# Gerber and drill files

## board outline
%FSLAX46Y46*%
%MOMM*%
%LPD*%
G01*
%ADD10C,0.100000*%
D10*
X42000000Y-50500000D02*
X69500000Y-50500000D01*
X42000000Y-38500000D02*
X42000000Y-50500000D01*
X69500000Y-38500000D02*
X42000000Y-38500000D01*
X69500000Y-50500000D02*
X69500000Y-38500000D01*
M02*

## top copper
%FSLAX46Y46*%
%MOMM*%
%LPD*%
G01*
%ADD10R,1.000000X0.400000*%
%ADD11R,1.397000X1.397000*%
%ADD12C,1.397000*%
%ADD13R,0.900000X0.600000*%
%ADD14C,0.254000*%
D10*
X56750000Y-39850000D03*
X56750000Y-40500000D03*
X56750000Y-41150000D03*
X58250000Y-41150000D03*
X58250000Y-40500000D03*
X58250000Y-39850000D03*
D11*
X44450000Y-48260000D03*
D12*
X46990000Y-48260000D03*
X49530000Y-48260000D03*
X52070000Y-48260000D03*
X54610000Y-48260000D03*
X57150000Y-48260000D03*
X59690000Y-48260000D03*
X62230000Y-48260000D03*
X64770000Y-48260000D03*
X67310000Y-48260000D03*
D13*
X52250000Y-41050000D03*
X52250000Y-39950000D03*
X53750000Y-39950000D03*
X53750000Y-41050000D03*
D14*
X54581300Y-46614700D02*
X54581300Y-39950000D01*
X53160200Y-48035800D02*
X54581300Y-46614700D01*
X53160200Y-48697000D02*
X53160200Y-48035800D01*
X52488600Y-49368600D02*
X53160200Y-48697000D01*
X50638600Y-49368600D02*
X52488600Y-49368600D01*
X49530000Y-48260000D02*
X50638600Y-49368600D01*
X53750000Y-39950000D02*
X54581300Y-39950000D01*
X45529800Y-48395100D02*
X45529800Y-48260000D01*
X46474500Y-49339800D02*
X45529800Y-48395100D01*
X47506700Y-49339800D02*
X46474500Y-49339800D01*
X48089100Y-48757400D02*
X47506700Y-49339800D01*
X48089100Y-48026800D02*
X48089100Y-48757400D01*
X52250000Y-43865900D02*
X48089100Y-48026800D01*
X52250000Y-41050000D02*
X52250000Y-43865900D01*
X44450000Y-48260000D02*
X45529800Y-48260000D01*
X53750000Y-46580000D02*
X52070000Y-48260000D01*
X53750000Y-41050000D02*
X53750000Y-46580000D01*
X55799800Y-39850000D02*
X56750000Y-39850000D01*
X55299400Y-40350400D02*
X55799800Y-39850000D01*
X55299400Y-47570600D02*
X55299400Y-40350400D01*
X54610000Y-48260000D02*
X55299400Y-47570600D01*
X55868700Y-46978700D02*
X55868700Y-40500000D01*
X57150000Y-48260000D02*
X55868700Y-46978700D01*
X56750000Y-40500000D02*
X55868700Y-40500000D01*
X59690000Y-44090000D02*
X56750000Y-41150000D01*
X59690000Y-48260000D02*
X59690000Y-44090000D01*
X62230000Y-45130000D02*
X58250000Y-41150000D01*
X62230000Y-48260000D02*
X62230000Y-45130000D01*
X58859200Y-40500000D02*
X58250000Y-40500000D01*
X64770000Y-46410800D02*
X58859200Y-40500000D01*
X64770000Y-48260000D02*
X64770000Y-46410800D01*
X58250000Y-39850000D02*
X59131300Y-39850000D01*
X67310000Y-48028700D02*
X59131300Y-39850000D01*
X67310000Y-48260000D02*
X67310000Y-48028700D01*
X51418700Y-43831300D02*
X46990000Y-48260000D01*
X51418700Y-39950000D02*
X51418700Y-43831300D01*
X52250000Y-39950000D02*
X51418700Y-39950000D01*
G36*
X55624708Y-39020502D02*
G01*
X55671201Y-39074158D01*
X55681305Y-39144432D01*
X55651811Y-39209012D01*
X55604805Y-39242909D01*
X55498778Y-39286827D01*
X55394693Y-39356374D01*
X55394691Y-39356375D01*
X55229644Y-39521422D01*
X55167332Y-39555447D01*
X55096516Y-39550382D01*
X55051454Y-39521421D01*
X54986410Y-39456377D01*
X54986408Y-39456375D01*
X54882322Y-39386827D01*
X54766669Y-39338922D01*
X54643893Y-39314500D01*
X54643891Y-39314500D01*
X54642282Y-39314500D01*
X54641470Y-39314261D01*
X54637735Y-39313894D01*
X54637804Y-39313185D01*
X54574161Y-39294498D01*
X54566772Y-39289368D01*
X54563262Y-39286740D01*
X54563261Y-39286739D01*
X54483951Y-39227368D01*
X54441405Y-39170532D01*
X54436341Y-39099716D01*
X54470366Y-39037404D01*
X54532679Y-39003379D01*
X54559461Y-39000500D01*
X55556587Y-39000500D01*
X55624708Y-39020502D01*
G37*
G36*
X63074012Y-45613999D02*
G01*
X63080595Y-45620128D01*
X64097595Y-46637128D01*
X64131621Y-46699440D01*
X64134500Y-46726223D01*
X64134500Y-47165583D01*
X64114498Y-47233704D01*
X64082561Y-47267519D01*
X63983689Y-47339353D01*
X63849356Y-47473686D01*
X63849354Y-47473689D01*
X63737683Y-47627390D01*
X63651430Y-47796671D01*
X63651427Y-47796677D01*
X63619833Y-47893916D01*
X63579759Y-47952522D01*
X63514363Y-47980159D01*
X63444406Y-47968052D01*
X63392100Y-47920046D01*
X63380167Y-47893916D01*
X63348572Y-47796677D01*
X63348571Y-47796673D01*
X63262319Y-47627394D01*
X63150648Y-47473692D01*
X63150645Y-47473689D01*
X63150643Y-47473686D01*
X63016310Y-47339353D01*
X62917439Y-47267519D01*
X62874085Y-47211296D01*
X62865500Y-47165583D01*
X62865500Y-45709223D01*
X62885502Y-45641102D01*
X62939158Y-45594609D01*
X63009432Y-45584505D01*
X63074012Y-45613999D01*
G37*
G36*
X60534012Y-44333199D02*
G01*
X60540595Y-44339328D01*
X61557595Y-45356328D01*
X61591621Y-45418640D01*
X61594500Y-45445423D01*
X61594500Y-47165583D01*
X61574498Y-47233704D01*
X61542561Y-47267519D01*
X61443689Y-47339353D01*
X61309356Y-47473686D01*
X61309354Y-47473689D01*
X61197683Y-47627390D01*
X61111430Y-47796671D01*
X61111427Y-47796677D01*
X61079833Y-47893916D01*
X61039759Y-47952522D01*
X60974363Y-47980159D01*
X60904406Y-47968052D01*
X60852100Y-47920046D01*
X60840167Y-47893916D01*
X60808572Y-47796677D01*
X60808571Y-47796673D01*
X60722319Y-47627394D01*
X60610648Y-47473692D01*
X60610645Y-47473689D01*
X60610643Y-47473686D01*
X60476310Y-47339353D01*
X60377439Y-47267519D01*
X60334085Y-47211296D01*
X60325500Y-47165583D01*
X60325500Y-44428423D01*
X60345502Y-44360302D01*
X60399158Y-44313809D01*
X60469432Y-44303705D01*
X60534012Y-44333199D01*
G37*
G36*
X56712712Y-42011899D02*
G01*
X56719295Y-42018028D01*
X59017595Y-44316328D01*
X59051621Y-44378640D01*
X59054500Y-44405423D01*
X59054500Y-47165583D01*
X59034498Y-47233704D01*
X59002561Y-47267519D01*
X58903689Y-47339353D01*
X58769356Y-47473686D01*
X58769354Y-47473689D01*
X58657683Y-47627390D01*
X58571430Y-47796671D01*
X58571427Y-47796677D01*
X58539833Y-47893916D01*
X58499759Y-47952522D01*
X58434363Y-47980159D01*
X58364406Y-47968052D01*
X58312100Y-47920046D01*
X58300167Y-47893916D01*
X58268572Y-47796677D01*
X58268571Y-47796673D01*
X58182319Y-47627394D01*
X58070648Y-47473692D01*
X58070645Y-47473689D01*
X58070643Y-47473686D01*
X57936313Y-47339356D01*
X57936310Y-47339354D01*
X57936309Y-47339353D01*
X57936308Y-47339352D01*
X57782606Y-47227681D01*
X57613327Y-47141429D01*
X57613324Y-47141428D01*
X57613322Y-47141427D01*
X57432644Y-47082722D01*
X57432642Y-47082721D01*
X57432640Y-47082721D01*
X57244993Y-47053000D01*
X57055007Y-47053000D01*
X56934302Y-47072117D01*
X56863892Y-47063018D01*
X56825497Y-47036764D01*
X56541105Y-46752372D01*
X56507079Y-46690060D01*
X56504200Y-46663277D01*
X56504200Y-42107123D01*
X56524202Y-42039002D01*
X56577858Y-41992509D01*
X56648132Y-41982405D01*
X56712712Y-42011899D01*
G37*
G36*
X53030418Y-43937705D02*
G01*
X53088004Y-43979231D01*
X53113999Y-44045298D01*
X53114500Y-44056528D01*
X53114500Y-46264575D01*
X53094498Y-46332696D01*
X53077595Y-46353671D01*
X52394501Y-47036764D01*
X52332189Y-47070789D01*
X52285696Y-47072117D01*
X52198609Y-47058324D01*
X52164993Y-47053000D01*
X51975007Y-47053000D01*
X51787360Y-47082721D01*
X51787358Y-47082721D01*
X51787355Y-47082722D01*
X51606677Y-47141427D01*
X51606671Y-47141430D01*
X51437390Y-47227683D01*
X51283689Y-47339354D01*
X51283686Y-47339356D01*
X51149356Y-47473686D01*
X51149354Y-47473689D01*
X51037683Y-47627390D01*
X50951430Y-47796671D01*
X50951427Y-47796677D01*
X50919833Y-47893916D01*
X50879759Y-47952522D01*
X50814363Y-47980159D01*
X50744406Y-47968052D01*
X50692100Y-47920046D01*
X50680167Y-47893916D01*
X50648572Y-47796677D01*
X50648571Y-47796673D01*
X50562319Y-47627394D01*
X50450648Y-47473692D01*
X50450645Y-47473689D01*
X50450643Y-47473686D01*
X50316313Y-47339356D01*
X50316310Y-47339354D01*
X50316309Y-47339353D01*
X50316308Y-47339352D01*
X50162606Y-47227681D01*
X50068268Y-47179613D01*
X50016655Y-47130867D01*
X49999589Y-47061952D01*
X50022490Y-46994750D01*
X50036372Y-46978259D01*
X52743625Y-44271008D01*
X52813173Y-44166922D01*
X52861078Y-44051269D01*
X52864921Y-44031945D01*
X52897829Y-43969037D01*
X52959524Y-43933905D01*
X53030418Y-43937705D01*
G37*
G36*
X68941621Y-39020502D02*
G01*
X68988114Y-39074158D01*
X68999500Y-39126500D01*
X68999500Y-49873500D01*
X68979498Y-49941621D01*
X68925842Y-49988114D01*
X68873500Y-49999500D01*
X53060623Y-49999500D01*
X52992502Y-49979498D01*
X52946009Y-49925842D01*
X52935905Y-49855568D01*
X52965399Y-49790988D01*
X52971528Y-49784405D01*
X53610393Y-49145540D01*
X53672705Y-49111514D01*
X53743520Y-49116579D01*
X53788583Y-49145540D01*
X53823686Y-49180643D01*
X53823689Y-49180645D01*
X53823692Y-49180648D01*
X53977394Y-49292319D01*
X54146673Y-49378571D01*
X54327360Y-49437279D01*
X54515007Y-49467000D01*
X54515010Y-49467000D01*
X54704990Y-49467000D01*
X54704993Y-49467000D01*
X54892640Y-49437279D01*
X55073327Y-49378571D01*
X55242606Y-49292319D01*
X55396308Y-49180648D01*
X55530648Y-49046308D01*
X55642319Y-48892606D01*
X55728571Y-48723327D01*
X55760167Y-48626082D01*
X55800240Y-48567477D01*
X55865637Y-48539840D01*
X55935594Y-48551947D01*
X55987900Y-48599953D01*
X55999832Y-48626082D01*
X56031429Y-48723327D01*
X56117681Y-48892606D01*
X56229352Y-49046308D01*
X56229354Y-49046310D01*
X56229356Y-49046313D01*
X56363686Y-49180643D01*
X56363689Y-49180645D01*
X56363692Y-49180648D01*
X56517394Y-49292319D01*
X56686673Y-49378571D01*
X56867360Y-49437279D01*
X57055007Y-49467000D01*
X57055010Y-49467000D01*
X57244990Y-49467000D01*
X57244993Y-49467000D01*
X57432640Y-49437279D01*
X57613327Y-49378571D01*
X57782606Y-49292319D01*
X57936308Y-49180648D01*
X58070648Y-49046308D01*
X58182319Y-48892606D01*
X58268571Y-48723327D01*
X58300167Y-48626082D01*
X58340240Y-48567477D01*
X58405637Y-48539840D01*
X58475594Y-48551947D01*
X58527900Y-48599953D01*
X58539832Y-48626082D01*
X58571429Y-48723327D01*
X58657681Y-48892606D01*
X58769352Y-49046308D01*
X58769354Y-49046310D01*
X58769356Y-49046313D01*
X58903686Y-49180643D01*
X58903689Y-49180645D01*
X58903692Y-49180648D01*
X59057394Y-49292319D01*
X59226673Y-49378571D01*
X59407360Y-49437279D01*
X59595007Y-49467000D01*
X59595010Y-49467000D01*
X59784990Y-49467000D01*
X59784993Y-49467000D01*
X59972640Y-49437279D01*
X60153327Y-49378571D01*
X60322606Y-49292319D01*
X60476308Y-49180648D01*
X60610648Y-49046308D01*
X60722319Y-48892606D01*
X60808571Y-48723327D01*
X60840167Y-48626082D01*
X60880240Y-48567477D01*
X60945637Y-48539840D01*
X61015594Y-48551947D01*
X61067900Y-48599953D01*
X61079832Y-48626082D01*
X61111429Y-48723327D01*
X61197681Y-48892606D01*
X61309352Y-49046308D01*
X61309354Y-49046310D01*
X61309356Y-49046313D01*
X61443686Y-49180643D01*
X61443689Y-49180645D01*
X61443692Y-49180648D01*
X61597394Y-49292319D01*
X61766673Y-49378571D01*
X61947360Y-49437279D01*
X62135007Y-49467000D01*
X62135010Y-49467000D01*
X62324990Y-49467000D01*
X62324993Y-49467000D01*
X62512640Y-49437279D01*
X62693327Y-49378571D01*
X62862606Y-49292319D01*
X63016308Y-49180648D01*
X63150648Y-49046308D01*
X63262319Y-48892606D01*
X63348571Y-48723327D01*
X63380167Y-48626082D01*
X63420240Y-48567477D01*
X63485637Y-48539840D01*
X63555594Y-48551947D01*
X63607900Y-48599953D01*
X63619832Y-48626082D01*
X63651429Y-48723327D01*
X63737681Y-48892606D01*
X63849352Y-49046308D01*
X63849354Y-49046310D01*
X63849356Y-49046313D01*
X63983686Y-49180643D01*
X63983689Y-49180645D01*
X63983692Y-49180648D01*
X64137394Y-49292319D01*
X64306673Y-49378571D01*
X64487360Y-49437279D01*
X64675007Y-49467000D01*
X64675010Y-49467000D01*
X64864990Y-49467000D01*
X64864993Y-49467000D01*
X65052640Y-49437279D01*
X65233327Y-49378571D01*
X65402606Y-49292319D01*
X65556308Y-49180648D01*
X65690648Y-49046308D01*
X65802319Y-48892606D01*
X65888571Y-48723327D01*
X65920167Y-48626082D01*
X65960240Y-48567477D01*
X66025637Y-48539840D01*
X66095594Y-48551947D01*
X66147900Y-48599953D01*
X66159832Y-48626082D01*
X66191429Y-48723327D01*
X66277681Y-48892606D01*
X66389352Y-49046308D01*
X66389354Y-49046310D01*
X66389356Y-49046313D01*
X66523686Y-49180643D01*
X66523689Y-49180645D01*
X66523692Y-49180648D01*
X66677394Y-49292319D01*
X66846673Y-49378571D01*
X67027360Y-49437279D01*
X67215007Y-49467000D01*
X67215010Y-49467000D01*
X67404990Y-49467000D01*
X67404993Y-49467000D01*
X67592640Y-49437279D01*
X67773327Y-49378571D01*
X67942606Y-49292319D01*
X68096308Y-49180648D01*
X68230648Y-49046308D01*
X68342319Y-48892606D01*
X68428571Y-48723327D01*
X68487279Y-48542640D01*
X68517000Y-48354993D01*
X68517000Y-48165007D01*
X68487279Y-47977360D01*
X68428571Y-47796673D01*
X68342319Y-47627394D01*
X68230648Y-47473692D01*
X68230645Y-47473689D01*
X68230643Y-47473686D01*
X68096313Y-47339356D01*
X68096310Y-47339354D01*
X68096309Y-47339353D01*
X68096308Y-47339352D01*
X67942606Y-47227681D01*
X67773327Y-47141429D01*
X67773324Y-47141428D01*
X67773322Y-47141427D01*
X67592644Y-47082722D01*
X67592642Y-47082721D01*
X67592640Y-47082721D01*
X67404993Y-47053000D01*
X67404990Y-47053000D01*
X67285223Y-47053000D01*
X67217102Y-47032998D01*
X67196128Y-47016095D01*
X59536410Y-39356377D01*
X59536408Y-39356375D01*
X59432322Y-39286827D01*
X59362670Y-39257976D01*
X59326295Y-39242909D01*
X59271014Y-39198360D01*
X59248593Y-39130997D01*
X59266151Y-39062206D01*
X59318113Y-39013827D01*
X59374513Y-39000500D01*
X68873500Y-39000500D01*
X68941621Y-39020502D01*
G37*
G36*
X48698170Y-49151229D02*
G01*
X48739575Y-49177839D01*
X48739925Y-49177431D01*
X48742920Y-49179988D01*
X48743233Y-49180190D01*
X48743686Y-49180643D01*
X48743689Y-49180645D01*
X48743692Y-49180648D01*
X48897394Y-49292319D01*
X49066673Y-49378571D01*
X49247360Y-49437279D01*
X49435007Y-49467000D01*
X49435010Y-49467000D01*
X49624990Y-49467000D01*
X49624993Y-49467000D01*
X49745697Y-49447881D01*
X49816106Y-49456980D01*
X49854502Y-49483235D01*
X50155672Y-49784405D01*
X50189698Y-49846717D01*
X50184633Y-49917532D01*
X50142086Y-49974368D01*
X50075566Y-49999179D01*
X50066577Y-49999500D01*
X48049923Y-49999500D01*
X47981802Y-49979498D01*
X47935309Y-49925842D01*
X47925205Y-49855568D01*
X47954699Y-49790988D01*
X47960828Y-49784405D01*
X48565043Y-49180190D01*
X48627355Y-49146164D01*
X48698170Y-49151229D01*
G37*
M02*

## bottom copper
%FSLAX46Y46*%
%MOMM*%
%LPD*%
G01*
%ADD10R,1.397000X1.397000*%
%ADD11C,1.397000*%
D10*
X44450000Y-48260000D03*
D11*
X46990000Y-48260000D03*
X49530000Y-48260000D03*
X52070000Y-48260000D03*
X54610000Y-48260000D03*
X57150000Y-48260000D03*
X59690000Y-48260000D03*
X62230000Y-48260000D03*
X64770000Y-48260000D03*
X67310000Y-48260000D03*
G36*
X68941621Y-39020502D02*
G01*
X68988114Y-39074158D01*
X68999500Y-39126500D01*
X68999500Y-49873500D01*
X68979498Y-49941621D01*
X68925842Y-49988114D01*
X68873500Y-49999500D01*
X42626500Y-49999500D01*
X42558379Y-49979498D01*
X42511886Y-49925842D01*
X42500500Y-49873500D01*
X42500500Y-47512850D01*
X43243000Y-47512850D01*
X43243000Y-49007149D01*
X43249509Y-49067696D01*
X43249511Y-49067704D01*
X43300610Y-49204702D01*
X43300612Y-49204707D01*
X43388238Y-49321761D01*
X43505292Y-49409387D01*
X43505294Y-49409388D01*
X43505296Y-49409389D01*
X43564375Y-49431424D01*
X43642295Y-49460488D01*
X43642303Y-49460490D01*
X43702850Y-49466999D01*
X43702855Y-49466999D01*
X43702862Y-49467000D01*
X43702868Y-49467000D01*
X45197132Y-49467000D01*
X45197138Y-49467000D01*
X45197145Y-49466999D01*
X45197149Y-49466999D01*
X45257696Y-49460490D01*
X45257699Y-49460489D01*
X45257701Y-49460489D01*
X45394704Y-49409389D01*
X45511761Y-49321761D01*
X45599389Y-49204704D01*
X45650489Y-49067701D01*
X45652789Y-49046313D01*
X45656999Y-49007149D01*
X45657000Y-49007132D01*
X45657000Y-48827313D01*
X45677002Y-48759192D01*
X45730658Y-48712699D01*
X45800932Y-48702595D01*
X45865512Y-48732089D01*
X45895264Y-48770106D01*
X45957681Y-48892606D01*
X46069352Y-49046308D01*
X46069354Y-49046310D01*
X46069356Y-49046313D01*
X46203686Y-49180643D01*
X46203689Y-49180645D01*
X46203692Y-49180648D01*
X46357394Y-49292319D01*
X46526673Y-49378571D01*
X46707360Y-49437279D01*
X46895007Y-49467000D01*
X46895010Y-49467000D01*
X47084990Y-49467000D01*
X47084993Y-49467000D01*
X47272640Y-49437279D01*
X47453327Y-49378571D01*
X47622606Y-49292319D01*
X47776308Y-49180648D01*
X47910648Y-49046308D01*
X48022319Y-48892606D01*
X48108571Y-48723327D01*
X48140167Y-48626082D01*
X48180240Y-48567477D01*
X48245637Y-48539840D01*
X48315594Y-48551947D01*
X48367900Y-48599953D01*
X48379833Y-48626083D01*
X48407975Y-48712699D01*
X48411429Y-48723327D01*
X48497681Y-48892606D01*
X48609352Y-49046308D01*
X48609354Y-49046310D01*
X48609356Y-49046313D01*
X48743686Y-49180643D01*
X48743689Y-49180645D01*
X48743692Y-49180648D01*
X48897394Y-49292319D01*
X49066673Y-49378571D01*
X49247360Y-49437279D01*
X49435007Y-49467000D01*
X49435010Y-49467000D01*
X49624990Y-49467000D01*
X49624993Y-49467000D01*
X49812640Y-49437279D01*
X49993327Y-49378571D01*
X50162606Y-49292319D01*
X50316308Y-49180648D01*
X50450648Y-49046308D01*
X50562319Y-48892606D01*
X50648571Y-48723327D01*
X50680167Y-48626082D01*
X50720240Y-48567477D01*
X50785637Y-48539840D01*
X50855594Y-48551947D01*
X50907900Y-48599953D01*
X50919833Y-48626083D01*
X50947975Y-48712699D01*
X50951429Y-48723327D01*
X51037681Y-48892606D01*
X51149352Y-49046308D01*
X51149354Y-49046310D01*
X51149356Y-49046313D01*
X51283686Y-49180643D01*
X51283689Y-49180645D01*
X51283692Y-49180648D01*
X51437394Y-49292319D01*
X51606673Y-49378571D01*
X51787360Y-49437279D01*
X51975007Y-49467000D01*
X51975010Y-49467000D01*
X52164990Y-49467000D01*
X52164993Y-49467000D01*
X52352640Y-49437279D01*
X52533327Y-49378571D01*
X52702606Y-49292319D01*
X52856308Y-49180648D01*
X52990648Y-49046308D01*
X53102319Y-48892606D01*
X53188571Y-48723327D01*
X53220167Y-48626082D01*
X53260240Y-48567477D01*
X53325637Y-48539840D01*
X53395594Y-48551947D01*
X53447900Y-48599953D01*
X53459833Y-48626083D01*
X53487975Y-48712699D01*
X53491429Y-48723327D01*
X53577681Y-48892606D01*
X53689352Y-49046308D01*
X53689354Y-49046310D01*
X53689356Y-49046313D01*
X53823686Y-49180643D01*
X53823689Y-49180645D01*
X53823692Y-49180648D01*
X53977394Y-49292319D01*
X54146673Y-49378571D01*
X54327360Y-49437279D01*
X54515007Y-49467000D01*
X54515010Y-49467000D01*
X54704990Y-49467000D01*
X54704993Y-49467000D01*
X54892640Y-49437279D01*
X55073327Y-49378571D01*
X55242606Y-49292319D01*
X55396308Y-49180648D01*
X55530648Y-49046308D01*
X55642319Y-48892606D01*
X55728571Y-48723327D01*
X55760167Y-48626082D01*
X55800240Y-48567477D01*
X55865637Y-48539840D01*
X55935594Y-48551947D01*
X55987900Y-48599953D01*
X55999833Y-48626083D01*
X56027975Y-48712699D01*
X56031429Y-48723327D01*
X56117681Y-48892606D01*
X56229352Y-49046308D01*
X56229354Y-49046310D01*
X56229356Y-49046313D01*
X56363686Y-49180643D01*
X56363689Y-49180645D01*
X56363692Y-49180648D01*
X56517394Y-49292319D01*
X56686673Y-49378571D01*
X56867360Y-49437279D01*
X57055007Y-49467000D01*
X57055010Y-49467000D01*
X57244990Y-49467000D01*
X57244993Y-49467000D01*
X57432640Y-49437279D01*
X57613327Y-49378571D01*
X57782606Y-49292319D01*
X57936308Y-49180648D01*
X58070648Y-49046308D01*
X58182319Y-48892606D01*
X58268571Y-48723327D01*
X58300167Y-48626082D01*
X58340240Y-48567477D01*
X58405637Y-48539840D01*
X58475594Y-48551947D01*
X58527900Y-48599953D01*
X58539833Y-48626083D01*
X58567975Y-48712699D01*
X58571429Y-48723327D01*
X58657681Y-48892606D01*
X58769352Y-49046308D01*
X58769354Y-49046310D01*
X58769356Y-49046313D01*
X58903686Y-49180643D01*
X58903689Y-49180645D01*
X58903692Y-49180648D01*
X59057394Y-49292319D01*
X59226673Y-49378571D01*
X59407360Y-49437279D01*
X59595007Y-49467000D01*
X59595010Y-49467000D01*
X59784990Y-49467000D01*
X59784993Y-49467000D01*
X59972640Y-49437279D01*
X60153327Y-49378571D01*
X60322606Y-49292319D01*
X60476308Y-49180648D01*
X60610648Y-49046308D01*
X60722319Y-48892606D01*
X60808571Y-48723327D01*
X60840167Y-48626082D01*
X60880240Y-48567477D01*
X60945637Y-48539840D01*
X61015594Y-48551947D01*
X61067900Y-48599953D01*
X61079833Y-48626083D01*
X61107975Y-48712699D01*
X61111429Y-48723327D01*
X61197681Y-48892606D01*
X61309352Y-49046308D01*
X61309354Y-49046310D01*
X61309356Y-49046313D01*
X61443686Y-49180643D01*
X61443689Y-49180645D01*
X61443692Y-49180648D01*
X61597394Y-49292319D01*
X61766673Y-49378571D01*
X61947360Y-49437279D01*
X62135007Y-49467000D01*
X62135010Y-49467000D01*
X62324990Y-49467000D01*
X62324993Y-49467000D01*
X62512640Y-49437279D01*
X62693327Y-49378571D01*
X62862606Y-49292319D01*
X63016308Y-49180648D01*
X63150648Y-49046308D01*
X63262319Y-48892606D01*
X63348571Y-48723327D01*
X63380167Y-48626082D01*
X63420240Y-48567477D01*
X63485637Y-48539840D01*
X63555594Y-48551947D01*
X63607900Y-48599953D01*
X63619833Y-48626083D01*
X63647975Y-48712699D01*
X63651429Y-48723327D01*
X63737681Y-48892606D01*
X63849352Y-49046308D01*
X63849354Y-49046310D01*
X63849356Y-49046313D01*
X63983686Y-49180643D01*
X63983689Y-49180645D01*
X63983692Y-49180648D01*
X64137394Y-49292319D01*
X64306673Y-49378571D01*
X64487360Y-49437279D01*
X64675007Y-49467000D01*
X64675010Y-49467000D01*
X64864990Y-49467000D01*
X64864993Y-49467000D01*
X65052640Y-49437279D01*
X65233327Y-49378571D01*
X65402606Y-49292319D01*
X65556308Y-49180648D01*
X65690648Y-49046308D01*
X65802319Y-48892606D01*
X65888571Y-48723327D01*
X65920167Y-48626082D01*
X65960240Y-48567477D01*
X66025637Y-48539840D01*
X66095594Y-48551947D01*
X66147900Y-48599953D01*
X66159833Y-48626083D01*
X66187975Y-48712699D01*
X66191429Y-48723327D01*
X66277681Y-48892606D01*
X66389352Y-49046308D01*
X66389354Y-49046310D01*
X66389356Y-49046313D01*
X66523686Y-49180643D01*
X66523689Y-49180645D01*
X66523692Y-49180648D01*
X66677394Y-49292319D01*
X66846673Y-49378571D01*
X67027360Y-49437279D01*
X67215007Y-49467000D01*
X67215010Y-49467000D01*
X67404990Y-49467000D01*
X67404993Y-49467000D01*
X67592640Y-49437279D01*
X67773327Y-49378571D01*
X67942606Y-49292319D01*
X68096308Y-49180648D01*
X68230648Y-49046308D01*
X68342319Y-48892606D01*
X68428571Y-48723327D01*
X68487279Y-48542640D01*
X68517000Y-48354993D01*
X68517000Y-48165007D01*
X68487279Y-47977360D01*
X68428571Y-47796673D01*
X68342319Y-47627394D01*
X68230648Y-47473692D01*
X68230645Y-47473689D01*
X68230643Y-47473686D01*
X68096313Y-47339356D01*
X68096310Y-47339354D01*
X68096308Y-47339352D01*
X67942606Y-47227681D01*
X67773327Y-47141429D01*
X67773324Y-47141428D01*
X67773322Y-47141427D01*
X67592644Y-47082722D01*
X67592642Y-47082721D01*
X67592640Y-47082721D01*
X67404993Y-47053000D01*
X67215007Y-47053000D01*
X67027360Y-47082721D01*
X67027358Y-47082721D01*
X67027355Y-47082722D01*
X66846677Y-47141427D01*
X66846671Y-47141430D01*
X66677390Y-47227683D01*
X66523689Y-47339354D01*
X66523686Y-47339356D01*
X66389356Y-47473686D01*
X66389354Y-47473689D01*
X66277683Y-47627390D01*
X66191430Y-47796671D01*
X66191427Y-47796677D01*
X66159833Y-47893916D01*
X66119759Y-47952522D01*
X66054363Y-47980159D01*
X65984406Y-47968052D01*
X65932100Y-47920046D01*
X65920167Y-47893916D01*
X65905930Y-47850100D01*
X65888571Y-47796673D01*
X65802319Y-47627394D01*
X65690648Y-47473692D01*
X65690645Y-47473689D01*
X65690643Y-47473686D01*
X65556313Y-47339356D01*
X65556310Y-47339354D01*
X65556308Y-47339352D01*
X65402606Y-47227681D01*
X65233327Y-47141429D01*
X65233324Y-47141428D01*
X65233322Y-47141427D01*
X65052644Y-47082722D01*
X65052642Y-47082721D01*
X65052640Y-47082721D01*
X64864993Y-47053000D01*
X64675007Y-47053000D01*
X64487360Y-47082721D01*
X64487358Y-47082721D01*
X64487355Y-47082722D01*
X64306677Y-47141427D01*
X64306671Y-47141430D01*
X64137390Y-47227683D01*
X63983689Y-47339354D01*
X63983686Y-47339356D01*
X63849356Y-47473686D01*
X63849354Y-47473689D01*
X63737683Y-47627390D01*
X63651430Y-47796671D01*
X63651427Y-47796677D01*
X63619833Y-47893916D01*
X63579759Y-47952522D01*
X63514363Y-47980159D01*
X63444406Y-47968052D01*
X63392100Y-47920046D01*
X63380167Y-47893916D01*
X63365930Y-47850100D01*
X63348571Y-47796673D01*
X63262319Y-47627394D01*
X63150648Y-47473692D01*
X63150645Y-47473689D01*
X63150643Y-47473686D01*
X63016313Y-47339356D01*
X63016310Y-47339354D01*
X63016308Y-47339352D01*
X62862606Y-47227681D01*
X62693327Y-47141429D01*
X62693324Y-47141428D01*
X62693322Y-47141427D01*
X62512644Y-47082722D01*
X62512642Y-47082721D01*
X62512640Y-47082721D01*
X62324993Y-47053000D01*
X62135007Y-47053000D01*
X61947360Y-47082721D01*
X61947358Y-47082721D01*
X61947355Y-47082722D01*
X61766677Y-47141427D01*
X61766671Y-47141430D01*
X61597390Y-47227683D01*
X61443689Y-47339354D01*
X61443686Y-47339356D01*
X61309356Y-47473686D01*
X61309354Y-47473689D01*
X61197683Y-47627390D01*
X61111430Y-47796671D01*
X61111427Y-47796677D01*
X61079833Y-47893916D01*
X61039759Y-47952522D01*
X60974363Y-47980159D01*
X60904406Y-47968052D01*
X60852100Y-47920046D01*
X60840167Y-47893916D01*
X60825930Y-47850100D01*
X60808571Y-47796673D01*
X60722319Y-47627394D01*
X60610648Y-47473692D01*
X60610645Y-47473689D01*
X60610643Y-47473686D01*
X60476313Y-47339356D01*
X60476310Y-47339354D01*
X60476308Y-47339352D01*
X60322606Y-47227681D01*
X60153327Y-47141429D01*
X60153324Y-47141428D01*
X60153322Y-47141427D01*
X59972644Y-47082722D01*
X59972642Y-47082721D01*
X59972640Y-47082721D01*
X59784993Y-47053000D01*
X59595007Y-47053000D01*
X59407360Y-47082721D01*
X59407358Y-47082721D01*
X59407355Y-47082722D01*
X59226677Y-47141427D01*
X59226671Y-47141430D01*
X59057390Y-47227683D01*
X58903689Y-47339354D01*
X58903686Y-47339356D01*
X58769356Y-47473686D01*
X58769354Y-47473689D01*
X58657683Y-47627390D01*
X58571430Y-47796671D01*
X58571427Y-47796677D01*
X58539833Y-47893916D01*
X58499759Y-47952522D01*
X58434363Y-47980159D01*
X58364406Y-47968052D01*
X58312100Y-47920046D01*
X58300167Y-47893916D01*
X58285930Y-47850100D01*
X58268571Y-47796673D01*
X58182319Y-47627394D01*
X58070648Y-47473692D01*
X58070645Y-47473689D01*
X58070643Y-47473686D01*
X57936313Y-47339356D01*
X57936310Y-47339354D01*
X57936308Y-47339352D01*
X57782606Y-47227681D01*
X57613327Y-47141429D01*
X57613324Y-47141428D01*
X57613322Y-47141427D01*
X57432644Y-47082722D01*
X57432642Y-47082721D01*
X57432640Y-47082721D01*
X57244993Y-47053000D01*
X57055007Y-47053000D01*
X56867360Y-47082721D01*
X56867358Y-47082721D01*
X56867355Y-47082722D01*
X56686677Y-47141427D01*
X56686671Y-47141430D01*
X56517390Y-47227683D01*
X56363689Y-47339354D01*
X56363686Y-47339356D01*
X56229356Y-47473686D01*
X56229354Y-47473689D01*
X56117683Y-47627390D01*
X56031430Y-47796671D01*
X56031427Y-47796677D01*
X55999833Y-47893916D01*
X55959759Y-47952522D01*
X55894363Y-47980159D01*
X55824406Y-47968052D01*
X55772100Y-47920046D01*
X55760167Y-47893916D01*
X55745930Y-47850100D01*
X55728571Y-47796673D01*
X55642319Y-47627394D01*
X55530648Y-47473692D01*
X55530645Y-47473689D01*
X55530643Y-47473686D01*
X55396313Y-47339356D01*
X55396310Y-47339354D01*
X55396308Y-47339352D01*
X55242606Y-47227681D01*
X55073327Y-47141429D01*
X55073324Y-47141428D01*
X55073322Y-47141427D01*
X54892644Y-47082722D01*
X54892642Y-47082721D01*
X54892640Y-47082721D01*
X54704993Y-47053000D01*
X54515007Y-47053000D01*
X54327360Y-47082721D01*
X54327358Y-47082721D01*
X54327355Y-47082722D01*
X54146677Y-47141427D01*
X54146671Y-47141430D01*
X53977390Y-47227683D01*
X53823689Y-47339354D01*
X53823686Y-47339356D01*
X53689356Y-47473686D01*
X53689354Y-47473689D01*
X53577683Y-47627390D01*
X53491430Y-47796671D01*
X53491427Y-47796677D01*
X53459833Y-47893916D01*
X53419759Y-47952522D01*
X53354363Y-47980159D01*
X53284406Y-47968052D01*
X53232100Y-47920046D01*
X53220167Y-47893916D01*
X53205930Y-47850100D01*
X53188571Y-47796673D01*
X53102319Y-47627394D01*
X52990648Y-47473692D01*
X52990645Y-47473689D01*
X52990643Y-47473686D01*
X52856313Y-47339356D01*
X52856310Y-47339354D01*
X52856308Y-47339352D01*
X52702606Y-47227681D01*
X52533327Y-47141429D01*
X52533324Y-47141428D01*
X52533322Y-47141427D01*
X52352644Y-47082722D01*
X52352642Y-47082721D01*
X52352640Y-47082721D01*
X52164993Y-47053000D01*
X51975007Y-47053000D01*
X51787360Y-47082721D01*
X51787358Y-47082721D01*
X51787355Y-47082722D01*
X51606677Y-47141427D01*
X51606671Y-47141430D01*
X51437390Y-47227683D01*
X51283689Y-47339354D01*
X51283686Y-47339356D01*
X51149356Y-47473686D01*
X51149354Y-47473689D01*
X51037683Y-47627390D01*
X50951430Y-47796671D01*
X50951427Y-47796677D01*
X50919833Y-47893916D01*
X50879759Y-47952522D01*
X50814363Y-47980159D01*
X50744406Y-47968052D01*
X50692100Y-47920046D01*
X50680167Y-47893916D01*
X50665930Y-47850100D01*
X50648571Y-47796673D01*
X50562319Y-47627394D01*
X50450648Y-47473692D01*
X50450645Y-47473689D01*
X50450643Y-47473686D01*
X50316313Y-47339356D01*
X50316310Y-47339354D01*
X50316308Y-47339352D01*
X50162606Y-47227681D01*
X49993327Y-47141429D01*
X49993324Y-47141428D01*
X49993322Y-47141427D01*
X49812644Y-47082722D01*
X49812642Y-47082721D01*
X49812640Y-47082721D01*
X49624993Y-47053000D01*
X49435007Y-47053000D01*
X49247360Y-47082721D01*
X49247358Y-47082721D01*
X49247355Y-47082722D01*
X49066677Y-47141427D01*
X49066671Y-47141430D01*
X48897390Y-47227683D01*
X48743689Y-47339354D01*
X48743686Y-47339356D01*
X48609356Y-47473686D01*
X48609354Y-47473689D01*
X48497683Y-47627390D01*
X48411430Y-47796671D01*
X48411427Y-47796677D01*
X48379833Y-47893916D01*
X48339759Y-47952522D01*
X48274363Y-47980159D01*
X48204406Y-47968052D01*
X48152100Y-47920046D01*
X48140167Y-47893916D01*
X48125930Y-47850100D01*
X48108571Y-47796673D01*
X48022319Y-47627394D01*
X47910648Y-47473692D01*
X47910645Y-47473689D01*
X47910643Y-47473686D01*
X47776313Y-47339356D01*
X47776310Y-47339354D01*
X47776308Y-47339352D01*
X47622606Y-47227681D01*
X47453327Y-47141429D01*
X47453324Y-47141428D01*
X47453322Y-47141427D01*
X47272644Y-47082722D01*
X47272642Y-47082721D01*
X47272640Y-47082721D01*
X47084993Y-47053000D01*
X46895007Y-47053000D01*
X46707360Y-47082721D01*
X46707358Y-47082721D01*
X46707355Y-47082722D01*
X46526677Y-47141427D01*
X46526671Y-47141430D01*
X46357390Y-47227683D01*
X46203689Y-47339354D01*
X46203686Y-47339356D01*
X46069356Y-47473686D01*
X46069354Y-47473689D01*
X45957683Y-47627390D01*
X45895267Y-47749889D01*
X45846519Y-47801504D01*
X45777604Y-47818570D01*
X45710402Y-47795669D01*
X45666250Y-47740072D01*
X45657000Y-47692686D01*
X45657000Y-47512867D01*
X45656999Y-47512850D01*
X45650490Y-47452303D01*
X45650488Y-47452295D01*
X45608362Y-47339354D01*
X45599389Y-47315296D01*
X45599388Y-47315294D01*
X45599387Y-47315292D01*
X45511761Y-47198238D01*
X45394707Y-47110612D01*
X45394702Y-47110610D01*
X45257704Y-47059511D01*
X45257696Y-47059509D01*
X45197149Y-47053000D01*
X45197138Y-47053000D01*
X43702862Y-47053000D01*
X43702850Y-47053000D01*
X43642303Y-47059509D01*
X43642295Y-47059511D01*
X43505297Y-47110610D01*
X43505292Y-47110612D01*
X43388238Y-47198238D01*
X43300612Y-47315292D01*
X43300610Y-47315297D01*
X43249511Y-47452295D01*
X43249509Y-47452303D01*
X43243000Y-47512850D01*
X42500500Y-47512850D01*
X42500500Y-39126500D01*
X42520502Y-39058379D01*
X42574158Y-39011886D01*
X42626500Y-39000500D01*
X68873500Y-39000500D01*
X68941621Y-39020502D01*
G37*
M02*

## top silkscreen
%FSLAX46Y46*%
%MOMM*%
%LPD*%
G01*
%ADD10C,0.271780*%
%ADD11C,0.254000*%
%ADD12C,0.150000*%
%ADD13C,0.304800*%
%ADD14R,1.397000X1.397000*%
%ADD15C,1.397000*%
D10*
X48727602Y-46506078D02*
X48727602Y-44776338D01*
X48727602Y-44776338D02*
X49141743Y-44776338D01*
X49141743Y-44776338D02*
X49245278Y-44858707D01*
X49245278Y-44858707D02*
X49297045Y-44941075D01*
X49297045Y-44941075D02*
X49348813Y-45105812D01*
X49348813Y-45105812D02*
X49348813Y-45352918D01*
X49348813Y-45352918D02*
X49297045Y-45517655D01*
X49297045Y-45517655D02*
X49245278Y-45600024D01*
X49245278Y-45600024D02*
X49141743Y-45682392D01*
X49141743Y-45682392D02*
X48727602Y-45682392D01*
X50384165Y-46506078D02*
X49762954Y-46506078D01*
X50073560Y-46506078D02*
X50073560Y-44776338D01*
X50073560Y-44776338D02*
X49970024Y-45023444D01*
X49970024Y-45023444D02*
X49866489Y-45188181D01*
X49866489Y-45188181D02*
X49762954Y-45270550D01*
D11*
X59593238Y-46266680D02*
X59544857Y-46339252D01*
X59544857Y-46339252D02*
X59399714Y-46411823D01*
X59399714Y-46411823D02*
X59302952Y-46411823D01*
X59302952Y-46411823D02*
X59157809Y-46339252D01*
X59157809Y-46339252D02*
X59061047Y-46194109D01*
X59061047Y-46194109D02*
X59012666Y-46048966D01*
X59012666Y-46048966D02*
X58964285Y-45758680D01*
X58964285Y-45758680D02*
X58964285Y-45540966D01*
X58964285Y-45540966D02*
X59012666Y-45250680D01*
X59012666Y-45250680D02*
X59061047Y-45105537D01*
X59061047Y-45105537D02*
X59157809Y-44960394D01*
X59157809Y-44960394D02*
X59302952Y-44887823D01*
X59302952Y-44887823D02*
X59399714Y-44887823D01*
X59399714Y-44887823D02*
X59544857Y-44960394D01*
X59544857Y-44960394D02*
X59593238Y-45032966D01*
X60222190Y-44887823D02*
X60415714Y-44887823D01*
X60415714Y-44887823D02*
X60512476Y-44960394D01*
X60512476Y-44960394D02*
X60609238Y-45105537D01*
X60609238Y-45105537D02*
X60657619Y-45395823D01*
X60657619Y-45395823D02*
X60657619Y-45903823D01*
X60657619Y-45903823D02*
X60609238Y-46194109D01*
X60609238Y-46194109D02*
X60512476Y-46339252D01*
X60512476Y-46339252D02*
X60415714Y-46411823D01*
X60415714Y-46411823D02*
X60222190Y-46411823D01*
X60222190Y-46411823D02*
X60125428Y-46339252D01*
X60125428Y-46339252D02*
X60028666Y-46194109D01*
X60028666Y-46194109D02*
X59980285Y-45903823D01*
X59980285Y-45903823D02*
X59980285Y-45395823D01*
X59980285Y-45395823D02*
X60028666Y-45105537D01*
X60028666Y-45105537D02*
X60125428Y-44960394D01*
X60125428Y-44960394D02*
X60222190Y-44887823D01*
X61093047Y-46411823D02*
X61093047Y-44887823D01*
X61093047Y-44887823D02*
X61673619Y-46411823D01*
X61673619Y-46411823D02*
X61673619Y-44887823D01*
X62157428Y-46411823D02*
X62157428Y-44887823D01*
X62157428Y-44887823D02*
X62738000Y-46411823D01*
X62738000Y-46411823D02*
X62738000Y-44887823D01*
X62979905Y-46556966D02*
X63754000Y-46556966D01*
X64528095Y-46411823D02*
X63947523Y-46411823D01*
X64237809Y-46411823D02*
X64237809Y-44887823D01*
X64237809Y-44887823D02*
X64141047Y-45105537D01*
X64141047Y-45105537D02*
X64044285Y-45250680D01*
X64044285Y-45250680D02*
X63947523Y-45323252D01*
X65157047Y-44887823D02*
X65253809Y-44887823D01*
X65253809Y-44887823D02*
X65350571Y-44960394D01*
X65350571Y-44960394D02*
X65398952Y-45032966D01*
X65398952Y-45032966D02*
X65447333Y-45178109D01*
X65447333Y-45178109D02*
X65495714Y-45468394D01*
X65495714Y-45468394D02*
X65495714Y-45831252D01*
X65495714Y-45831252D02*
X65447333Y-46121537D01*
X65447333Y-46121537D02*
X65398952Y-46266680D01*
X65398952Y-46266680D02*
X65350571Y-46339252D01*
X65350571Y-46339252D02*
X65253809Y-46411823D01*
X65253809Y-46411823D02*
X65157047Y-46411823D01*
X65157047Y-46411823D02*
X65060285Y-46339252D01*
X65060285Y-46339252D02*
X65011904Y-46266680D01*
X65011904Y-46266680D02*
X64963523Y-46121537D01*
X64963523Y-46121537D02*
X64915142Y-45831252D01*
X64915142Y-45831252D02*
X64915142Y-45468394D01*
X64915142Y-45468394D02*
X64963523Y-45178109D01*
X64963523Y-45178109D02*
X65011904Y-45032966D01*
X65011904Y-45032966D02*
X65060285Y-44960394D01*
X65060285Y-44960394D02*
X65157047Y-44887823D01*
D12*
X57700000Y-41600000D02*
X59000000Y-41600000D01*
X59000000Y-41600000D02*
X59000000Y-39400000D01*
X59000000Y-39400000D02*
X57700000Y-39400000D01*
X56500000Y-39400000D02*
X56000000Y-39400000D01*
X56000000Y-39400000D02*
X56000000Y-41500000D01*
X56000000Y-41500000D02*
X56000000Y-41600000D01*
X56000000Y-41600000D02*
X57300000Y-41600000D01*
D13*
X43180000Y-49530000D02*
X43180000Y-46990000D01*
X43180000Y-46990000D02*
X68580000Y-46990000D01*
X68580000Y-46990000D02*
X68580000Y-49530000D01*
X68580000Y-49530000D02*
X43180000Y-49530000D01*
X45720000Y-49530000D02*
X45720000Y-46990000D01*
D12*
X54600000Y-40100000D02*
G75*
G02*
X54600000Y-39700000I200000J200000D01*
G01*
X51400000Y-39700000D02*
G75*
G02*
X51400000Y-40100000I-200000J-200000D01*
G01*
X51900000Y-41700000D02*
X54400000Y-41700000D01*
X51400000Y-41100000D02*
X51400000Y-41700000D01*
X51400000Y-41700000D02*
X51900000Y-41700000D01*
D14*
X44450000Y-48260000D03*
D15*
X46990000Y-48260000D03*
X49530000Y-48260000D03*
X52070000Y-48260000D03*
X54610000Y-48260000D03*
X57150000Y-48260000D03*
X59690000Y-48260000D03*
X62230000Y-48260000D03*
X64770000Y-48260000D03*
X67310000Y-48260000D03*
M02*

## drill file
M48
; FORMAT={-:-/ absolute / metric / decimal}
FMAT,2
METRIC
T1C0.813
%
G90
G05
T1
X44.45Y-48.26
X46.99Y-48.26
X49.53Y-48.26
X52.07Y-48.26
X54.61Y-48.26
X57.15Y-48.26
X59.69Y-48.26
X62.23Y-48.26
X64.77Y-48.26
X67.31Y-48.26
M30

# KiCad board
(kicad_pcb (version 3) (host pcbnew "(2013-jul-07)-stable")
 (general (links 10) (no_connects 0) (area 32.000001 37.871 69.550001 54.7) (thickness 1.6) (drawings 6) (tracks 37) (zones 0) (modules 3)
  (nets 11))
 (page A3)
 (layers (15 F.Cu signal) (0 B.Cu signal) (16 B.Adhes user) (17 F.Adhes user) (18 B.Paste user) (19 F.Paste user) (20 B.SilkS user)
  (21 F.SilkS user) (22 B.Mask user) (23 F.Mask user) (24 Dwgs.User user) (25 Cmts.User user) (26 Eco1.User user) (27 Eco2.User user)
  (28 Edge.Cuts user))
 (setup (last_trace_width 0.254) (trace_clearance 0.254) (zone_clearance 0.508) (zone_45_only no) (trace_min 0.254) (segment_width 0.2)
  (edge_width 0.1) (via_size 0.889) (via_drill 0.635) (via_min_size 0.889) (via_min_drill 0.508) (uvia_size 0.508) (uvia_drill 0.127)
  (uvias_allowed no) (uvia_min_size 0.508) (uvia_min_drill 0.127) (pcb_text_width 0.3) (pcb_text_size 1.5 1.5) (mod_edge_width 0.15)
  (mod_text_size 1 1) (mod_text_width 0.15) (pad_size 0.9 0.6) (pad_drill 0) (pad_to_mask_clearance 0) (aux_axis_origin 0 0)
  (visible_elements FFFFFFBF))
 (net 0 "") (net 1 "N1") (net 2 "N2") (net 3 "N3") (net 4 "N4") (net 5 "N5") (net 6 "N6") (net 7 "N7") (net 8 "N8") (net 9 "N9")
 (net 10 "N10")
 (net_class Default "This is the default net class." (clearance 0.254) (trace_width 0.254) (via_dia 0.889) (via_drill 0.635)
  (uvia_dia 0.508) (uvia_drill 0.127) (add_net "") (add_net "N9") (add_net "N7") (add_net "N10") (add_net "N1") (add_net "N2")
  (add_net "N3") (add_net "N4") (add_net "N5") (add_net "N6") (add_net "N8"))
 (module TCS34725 (layer F.Cu) (at 57.5 40.5 180)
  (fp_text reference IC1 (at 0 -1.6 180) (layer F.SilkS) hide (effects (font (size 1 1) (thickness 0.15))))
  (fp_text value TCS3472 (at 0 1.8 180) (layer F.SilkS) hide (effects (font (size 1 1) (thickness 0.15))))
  (fp_line (start -0.2 -1.1) (end -1.5 -1.1) (layer F.SilkS) (width 0.15))
  (fp_line (start -1.5 -1.1) (end -1.5 1.1) (layer F.SilkS) (width 0.15))
  (fp_line (start -1.5 1.1) (end -0.2 1.1) (layer F.SilkS) (width 0.15))
  (fp_line (start 1 1.1) (end 1.5 1.1) (layer F.SilkS) (width 0.15))
  (fp_line (start 1.5 1.1) (end 1.5 -1) (layer F.SilkS) (width 0.15))
  (fp_line (start 1.5 -1) (end 1.5 -1.1) (layer F.SilkS) (width 0.15))
  (fp_line (start 1.5 -1.1) (end 0.2 -1.1) (layer F.SilkS) (width 0.15))
  (pad 1 smd rect (at 0.75 0.65 180) (size 1 0.4) (layers F.Cu F.Paste F.Mask) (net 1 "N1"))
  (pad 2 smd rect (at 0.75 0 180) (size 1 0.4) (layers F.Cu F.Paste F.Mask) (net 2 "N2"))
  (pad 3 smd rect (at 0.75 -0.65 180) (size 1 0.4) (layers F.Cu F.Paste F.Mask) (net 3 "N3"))
  (pad 4 smd rect (at -0.75 -0.65 180) (size 1 0.4) (layers F.Cu F.Paste F.Mask) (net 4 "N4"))
  (pad 5 smd rect (at -0.75 0 180) (size 1 0.4) (layers F.Cu F.Paste F.Mask) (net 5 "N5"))
  (pad 6 smd rect (at -0.75 0.65 180) (size 1 0.4) (layers F.Cu F.Paste F.Mask) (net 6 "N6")))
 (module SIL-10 (layer F.Cu) (at 55.88 48.26)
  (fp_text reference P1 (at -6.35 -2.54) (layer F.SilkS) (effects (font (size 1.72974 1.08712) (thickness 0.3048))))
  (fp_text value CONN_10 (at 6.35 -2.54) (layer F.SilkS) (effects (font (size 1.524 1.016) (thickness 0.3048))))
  (fp_line (start -12.7 1.27) (end -12.7 -1.27) (layer F.SilkS) (width 0.3048))
  (fp_line (start -12.7 -1.27) (end 12.7 -1.27) (layer F.SilkS) (width 0.3048))
  (fp_line (start 12.7 -1.27) (end 12.7 1.27) (layer F.SilkS) (width 0.3048))
  (fp_line (start 12.7 1.27) (end -12.7 1.27) (layer F.SilkS) (width 0.3048))
  (fp_line (start -10.16 1.27) (end -10.16 -1.27) (layer F.SilkS) (width 0.3048))
  (pad 1 thru_hole rect (at -11.43 0) (size 1.397 1.397) (drill 0.8128) (layers *.Cu *.Mask F.SilkS) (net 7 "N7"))
  (pad 2 thru_hole circle (at -8.89 0) (size 1.397 1.397) (drill 0.8128) (layers *.Cu *.Mask F.SilkS) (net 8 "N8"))
  (pad 3 thru_hole circle (at -6.35 0) (size 1.397 1.397) (drill 0.8128) (layers *.Cu *.Mask F.SilkS) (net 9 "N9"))
  (pad 4 thru_hole circle (at -3.81 0) (size 1.397 1.397) (drill 0.8128) (layers *.Cu *.Mask F.SilkS) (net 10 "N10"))
  (pad 5 thru_hole circle (at -1.27 0) (size 1.397 1.397) (drill 0.8128) (layers *.Cu *.Mask F.SilkS) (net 1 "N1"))
  (pad 6 thru_hole circle (at 1.27 0) (size 1.397 1.397) (drill 0.8128) (layers *.Cu *.Mask F.SilkS) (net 2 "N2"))
  (pad 7 thru_hole circle (at 3.81 0) (size 1.397 1.397) (drill 0.8128) (layers *.Cu *.Mask F.SilkS) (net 3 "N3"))
  (pad 8 thru_hole circle (at 6.35 0) (size 1.397 1.397) (drill 0.8128) (layers *.Cu *.Mask F.SilkS) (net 4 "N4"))
  (pad 9 thru_hole circle (at 8.89 0) (size 1.397 1.397) (drill 0.8128) (layers *.Cu *.Mask F.SilkS) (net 5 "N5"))
  (pad 10 thru_hole circle (at 11.43 0) (size 1.397 1.397) (drill 0.8128) (layers *.Cu *.Mask F.SilkS) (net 6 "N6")))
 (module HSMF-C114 (layer F.Cu) (at 53 40.5)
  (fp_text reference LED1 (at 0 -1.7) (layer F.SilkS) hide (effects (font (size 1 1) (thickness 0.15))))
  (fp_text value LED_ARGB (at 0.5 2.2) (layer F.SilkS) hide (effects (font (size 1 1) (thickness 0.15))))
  (fp_arc (start 1.8 -0.6) (end 1.6 -0.4) (angle 90) (layer F.SilkS) (width 0.15))
  (fp_arc (start -1.8 -0.6) (end -1.6 -0.8) (angle 90) (layer F.SilkS) (width 0.15))
  (fp_line (start -1.1 1.2) (end 1.4 1.2) (layer F.SilkS) (width 0.15))
  (fp_line (start -1.6 0.6) (end -1.6 1.2) (layer F.SilkS) (width 0.15))
  (fp_line (start -1.6 1.2) (end -1.1 1.2) (layer F.SilkS) (width 0.15))
  (pad 1 smd rect (at -0.75 0.55) (size 0.9 0.6) (layers F.Cu F.Paste F.Mask) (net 7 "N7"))
  (pad 2 smd rect (at -0.75 -0.55) (size 0.9 0.6) (layers F.Cu F.Paste F.Mask) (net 8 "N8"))
  (pad 3 smd rect (at 0.75 -0.55) (size 0.9 0.6) (layers F.Cu F.Paste F.Mask) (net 9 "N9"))
  (pad 4 smd rect (at 0.75 0.55) (size 0.9 0.6) (layers F.Cu F.Paste F.Mask) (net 10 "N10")))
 (gr_line (start 42 50.5) (end 69.5 50.5) (angle 90) (layer Edge.Cuts) (width 0.1))
 (gr_line (start 42 38.5) (end 42 50.5) (angle 90) (layer Edge.Cuts) (width 0.1))
 (gr_line (start 69.5 38.5) (end 42 38.5) (angle 90) (layer Edge.Cuts) (width 0.1))
 (gr_line (start 69.5 50.5) (end 69.5 38.5) (angle 90) (layer Edge.Cuts) (width 0.1))
 (segment (start 54.5813 46.6147) (end 54.5813 39.95) (width 0.254) (layer F.Cu) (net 9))
 (segment (start 53.1602 48.0358) (end 54.5813 46.6147) (width 0.254) (layer F.Cu) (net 9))
 (segment (start 53.1602 48.697) (end 53.1602 48.0358) (width 0.254) (layer F.Cu) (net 9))
 (segment (start 52.4886 49.3686) (end 53.1602 48.697) (width 0.254) (layer F.Cu) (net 9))
 (segment (start 50.6386 49.3686) (end 52.4886 49.3686) (width 0.254) (layer F.Cu) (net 9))
 (segment (start 49.53 48.26) (end 50.6386 49.3686) (width 0.254) (layer F.Cu) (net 9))
 (segment (start 53.75 39.95) (end 54.5813 39.95) (width 0.254) (layer F.Cu) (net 9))
 (segment (start 45.5298 48.3951) (end 45.5298 48.26) (width 0.254) (layer F.Cu) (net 7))
 (segment (start 46.4745 49.3398) (end 45.5298 48.3951) (width 0.254) (layer F.Cu) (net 7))
 (segment (start 47.5067 49.3398) (end 46.4745 49.3398) (width 0.254) (layer F.Cu) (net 7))
 (segment (start 48.0891 48.7574) (end 47.5067 49.3398) (width 0.254) (layer F.Cu) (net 7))
 (segment (start 48.0891 48.0268) (end 48.0891 48.7574) (width 0.254) (layer F.Cu) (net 7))
 (segment (start 52.25 43.8659) (end 48.0891 48.0268) (width 0.254) (layer F.Cu) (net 7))
 (segment (start 52.25 41.05) (end 52.25 43.8659) (width 0.254) (layer F.Cu) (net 7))
 (segment (start 44.45 48.26) (end 45.5298 48.26) (width 0.254) (layer F.Cu) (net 7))
 (segment (start 53.75 46.58) (end 52.07 48.26) (width 0.254) (layer F.Cu) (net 10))
 (segment (start 53.75 41.05) (end 53.75 46.58) (width 0.254) (layer F.Cu) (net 10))
 (segment (start 55.7998 39.85) (end 56.75 39.85) (width 0.254) (layer F.Cu) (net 1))
 (segment (start 55.2994 40.3504) (end 55.7998 39.85) (width 0.254) (layer F.Cu) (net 1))
 (segment (start 55.2994 47.5706) (end 55.2994 40.3504) (width 0.254) (layer F.Cu) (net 1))
 (segment (start 54.61 48.26) (end 55.2994 47.5706) (width 0.254) (layer F.Cu) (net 1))
 (segment (start 55.8687 46.9787) (end 55.8687 40.5) (width 0.254) (layer F.Cu) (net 2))
 (segment (start 57.15 48.26) (end 55.8687 46.9787) (width 0.254) (layer F.Cu) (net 2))
 (segment (start 56.75 40.5) (end 55.8687 40.5) (width 0.254) (layer F.Cu) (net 2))
 (segment (start 59.69 44.09) (end 56.75 41.15) (width 0.254) (layer F.Cu) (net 3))
 (segment (start 59.69 48.26) (end 59.69 44.09) (width 0.254) (layer F.Cu) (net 3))
 (segment (start 62.23 45.13) (end 58.25 41.15) (width 0.254) (layer F.Cu) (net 4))
 (segment (start 62.23 48.26) (end 62.23 45.13) (width 0.254) (layer F.Cu) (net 4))
 (segment (start 58.8592 40.5) (end 58.25 40.5) (width 0.254) (layer F.Cu) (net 5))
 (segment (start 64.77 46.4108) (end 58.8592 40.5) (width 0.254) (layer F.Cu) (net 5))
 (segment (start 64.77 48.26) (end 64.77 46.4108) (width 0.254) (layer F.Cu) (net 5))
 (segment (start 58.25 39.85) (end 59.1313 39.85) (width 0.254) (layer F.Cu) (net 6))
 (segment (start 67.31 48.0287) (end 59.1313 39.85) (width 0.254) (layer F.Cu) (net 6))
 (segment (start 67.31 48.26) (end 67.31 48.0287) (width 0.254) (layer F.Cu) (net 6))
 (segment (start 51.4187 43.8313) (end 46.99 48.26) (width 0.254) (layer F.Cu) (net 8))
 (segment (start 51.4187 39.95) (end 51.4187 43.8313) (width 0.254) (layer F.Cu) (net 8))
 (segment (start 52.25 39.95) (end 51.4187 39.95) (width 0.254) (layer F.Cu) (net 8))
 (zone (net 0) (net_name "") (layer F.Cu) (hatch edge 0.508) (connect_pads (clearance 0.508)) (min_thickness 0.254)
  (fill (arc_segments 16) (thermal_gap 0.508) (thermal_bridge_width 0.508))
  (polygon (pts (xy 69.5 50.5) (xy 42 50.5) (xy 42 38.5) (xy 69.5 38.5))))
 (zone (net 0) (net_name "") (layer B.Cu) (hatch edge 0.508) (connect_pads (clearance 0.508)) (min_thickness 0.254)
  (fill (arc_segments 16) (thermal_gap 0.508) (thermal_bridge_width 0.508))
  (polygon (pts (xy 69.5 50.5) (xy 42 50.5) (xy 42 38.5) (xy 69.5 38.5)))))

